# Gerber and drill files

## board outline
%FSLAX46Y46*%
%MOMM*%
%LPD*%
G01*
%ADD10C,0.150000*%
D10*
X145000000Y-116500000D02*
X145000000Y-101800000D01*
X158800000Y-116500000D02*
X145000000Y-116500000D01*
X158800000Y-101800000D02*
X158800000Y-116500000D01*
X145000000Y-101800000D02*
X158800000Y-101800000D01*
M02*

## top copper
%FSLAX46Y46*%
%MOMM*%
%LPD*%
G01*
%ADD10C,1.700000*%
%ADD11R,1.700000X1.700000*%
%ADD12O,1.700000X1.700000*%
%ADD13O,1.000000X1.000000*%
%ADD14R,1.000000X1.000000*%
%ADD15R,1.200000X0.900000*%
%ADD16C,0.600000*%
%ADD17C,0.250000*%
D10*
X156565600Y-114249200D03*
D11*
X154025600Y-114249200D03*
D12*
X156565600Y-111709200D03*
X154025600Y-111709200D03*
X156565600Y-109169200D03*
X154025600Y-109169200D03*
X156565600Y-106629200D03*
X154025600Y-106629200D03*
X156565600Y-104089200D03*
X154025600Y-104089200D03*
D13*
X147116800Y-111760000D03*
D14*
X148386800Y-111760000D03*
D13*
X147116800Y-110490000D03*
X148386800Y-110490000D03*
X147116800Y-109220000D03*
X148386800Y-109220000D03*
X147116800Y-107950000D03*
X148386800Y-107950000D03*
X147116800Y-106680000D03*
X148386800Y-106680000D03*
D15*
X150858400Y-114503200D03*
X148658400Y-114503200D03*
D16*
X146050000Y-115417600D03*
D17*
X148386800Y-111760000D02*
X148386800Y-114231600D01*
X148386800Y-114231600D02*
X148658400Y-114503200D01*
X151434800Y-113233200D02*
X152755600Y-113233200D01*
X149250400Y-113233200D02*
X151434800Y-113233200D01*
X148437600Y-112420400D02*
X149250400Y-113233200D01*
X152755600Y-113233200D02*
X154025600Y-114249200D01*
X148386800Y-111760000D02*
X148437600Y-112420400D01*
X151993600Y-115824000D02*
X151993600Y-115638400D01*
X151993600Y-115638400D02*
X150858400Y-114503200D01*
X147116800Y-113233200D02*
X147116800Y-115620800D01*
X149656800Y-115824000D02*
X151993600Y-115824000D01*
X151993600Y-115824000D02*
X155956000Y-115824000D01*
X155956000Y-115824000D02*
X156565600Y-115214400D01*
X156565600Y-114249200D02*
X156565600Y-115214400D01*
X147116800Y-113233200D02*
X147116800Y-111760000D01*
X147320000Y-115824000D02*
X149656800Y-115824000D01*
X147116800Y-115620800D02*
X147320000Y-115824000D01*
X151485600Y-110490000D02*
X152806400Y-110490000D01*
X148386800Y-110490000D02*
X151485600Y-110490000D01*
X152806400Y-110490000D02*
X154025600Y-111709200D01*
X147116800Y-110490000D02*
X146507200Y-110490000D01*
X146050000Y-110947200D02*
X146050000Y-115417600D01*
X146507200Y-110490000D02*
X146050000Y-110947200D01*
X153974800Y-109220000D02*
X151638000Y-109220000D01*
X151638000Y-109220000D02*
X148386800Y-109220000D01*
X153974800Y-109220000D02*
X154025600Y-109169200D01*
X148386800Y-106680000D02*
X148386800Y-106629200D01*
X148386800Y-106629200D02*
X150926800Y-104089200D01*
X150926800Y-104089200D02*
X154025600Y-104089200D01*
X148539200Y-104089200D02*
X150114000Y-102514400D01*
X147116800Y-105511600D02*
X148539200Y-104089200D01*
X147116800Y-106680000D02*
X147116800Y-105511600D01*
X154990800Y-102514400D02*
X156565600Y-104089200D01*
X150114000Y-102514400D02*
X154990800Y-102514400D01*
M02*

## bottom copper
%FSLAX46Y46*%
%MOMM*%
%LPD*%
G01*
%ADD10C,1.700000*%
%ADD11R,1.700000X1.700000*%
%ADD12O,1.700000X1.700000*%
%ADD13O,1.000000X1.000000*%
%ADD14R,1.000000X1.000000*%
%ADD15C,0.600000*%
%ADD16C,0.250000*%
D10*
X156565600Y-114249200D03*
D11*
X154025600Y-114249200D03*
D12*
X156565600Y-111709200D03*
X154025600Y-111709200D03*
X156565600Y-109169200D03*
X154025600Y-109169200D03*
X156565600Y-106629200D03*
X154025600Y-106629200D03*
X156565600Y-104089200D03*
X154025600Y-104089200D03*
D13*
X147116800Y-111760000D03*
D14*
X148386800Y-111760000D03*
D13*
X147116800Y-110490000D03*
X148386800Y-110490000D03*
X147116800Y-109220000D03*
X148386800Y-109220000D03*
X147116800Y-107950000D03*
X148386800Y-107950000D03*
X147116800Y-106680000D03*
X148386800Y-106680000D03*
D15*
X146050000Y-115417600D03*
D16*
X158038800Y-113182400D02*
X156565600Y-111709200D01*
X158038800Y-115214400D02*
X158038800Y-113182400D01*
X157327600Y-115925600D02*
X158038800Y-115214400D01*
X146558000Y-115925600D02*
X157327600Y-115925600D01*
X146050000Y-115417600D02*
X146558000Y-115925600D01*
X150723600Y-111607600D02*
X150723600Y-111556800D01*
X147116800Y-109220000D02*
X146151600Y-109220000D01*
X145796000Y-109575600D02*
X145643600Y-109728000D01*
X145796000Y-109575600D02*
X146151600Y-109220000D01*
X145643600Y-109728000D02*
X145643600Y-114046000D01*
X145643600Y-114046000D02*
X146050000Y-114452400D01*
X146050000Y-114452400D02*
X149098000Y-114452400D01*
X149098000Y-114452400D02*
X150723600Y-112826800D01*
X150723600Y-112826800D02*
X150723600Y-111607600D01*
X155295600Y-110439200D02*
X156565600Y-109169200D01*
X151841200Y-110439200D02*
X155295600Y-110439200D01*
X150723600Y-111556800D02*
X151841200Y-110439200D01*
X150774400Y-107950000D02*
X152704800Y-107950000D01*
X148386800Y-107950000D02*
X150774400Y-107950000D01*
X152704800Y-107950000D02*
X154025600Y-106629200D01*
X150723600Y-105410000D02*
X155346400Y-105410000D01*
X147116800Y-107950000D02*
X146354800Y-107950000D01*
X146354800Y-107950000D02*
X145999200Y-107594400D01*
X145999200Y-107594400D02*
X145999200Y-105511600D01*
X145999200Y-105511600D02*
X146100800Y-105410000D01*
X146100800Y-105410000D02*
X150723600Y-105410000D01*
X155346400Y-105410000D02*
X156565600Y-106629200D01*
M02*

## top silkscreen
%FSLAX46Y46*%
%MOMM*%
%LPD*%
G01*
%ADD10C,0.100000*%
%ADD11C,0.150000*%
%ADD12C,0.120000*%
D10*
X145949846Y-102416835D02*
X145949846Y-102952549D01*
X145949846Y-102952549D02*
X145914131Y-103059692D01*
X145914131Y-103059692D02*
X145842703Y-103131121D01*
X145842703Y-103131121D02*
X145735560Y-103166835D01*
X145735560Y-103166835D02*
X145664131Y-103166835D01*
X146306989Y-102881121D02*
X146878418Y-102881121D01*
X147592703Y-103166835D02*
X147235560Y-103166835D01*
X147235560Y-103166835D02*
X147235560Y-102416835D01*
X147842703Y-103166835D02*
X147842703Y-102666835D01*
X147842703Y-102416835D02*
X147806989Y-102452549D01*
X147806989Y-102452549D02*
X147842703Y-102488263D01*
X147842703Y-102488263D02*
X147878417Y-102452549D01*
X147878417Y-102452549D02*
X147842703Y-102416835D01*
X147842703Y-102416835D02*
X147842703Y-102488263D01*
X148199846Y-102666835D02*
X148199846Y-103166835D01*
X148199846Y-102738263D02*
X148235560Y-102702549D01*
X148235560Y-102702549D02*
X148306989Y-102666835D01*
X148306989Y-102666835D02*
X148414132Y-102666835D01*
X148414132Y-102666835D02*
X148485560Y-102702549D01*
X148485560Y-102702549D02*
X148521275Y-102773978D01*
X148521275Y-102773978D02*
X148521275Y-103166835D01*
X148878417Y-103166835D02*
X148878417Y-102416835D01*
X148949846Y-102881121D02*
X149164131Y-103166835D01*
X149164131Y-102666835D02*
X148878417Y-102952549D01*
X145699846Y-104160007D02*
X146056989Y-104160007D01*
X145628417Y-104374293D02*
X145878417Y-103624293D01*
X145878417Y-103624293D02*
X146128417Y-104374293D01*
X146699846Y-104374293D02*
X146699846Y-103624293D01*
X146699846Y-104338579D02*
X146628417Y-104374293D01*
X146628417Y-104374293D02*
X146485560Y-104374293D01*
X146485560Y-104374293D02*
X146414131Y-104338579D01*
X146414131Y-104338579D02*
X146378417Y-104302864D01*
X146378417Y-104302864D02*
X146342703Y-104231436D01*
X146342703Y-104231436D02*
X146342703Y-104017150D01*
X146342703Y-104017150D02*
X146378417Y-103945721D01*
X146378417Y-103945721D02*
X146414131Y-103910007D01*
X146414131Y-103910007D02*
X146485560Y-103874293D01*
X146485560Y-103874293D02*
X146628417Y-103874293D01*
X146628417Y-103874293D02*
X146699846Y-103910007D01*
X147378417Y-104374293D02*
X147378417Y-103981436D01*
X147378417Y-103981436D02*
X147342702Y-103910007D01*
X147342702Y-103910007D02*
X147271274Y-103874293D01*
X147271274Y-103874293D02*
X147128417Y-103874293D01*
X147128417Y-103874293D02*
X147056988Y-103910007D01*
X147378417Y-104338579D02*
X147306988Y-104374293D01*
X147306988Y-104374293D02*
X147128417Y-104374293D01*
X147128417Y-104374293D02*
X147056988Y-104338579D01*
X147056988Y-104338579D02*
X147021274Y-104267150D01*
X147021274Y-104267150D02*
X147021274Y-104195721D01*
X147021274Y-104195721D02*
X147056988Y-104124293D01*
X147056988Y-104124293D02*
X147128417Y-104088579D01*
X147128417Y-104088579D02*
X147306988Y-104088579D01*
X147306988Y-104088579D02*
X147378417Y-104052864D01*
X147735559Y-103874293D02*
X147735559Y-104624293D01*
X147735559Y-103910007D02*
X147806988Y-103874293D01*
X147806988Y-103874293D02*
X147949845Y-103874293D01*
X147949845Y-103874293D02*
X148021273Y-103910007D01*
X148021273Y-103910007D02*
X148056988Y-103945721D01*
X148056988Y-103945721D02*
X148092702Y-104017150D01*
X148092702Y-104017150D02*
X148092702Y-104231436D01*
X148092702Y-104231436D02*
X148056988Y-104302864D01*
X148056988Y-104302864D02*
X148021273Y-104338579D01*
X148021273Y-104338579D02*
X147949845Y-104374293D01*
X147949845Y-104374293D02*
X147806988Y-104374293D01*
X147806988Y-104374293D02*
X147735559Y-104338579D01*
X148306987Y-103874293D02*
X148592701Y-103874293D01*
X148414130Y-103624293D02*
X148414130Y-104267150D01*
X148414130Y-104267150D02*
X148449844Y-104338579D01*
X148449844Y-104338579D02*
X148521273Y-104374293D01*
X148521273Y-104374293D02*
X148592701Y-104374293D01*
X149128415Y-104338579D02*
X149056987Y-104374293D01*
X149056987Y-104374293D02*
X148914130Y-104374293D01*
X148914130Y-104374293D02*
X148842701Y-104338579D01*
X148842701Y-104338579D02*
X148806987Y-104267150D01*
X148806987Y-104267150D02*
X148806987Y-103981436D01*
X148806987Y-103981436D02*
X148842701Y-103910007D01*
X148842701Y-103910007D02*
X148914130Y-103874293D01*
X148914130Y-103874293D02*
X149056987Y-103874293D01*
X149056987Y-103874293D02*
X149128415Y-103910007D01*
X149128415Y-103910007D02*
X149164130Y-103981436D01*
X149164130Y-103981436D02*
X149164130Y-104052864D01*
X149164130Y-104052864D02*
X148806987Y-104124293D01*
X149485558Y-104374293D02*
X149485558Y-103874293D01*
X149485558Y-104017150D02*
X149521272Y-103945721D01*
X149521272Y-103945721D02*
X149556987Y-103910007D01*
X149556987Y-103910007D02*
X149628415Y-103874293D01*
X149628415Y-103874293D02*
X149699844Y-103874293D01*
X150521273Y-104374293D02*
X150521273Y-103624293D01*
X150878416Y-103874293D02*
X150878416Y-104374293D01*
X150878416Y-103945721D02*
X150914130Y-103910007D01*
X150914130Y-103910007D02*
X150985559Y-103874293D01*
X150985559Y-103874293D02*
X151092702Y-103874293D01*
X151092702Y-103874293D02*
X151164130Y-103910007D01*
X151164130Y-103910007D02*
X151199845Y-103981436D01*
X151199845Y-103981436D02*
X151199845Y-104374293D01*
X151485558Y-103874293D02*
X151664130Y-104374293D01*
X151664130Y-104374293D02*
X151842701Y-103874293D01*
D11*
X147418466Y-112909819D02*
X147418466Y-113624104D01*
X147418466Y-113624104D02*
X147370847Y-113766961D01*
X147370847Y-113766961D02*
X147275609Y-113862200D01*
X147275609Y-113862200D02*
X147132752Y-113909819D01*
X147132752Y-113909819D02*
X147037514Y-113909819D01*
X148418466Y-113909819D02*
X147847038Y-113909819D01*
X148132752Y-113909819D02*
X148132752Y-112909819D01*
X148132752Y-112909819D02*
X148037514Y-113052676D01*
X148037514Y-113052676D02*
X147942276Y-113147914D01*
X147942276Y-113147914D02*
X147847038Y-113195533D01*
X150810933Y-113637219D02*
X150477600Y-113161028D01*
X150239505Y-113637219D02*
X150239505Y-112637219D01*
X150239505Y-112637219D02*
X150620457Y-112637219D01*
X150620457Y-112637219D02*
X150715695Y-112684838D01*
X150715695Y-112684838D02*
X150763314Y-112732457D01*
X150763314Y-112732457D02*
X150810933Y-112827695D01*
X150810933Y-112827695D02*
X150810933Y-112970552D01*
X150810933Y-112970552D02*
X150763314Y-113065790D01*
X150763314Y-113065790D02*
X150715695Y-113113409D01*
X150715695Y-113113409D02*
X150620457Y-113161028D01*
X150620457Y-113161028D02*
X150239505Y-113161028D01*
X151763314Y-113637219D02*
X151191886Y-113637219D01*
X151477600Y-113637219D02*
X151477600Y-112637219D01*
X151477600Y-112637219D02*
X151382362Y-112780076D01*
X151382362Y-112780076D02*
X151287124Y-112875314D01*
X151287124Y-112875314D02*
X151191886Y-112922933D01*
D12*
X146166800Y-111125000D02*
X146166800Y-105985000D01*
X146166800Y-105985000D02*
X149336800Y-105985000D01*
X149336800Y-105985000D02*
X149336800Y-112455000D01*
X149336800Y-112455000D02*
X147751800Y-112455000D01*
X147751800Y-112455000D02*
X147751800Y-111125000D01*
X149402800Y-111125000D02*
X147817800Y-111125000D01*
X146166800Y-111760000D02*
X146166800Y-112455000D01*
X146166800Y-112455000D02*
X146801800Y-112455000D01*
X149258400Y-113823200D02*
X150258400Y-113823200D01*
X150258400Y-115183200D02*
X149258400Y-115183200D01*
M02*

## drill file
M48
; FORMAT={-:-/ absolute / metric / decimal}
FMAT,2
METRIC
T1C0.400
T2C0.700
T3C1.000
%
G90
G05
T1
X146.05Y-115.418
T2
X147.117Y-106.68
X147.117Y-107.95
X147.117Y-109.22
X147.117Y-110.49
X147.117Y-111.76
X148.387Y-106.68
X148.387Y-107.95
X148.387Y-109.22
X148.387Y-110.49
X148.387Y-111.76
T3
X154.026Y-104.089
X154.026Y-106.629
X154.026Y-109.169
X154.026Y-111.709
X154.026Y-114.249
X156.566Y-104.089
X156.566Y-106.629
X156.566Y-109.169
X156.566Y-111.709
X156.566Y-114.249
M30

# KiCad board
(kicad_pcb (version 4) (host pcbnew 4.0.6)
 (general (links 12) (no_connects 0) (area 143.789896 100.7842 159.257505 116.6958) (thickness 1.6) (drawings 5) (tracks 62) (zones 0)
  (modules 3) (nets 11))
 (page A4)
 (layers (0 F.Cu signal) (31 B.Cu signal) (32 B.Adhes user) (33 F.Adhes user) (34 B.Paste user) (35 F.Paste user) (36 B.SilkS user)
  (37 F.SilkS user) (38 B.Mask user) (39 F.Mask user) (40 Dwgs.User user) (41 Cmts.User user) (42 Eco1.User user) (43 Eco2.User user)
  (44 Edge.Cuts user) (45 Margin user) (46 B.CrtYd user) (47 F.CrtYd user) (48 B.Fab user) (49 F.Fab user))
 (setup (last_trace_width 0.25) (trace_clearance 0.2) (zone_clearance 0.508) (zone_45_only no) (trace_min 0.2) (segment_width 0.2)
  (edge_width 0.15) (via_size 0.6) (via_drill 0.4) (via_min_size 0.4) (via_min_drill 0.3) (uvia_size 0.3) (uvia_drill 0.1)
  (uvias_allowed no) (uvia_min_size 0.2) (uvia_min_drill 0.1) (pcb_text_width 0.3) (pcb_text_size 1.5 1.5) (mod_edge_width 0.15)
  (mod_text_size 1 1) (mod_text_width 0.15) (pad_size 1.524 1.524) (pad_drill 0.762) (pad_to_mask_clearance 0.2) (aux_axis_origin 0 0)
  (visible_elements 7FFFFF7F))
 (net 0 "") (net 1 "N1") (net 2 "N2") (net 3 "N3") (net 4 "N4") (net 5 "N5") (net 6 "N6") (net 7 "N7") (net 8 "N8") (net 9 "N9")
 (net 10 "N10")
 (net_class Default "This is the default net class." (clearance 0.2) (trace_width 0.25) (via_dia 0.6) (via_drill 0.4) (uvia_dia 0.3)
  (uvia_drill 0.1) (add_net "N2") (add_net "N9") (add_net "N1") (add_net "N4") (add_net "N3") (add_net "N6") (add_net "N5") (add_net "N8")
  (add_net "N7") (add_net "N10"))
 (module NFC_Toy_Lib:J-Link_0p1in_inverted (layer B.Cu) (at 156.5656 114.2492)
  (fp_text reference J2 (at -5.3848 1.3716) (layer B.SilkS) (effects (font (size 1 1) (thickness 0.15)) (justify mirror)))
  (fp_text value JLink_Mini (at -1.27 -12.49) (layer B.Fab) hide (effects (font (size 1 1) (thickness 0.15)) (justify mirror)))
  (pad 2 thru_hole circle (at 0 0) (size 1.7 1.7) (drill 1) (layers *.Cu *.Mask) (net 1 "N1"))
  (pad 1 thru_hole rect (at -2.54 0) (size 1.7 1.7) (drill 1) (layers *.Cu *.Mask) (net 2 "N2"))
  (pad 4 thru_hole oval (at 0 -2.54) (size 1.7 1.7) (drill 1) (layers *.Cu *.Mask) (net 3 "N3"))
  (pad 3 thru_hole oval (at -2.54 -2.54) (size 1.7 1.7) (drill 1) (layers *.Cu *.Mask) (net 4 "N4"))
  (pad 6 thru_hole oval (at 0 -5.08) (size 1.7 1.7) (drill 1) (layers *.Cu *.Mask) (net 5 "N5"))
  (pad 5 thru_hole oval (at -2.54 -5.08) (size 1.7 1.7) (drill 1) (layers *.Cu *.Mask) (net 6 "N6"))
  (pad 8 thru_hole oval (at 0 -7.62) (size 1.7 1.7) (drill 1) (layers *.Cu *.Mask) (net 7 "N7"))
  (pad 7 thru_hole oval (at -2.54 -7.62) (size 1.7 1.7) (drill 1) (layers *.Cu *.Mask) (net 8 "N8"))
  (pad 10 thru_hole oval (at 0 -10.16) (size 1.7 1.7) (drill 1) (layers *.Cu *.Mask) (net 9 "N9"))
  (pad 9 thru_hole oval (at -2.54 -10.16) (size 1.7 1.7) (drill 1) (layers *.Cu *.Mask) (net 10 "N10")))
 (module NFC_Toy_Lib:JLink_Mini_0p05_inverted (layer F.Cu) (at 147.1168 111.76 180)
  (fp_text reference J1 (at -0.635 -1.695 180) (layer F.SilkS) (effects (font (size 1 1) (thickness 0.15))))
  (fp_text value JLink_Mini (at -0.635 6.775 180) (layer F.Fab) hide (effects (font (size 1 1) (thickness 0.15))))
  (fp_line (start 0.95 0.635) (end 0.95 5.775) (layer F.SilkS) (width 0.12))
  (fp_line (start 0.95 5.775) (end -2.22 5.775) (layer F.SilkS) (width 0.12))
  (fp_line (start -2.22 5.775) (end -2.22 -0.695) (layer F.SilkS) (width 0.12))
  (fp_line (start -2.22 -0.695) (end -0.635 -0.695) (layer F.SilkS) (width 0.12))
  (fp_line (start -0.635 -0.695) (end -0.635 0.635) (layer F.SilkS) (width 0.12))
  (fp_line (start -2.286 0.635) (end -0.701 0.635) (layer F.SilkS) (width 0.12))
  (fp_line (start 0.95 0) (end 0.95 -0.695) (layer F.SilkS) (width 0.12))
  (fp_line (start 0.95 -0.695) (end 0.315 -0.695) (layer F.SilkS) (width 0.12))
  (pad 2 thru_hole oval (at 0 0 180) (size 1 1) (drill 0.7) (layers *.Cu *.Mask) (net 1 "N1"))
  (pad 1 thru_hole rect (at -1.27 0 180) (size 1 1) (drill 0.7) (layers *.Cu *.Mask) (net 2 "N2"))
  (pad 4 thru_hole oval (at 0 1.27 180) (size 1 1) (drill 0.7) (layers *.Cu *.Mask) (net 3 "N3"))
  (pad 3 thru_hole oval (at -1.27 1.27 180) (size 1 1) (drill 0.7) (layers *.Cu *.Mask) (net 4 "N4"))
  (pad 6 thru_hole oval (at 0 2.54 180) (size 1 1) (drill 0.7) (layers *.Cu *.Mask) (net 5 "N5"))
  (pad 5 thru_hole oval (at -1.27 2.54 180) (size 1 1) (drill 0.7) (layers *.Cu *.Mask) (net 6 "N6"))
  (pad 8 thru_hole oval (at 0 3.81 180) (size 1 1) (drill 0.7) (layers *.Cu *.Mask) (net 7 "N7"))
  (pad 7 thru_hole oval (at -1.27 3.81 180) (size 1 1) (drill 0.7) (layers *.Cu *.Mask) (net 8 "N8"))
  (pad 10 thru_hole oval (at 0 5.08 180) (size 1 1) (drill 0.7) (layers *.Cu *.Mask) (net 9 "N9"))
  (pad 9 thru_hole oval (at -1.27 5.08 180) (size 1 1) (drill 0.7) (layers *.Cu *.Mask) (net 10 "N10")))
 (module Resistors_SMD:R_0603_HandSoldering (layer F.Cu) (at 149.7584 114.5032 180)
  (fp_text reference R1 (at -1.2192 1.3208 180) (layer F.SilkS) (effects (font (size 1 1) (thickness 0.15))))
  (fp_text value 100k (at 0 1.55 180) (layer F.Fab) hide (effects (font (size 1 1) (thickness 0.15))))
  (fp_line (start 0.5 0.68) (end -0.5 0.68) (layer F.SilkS) (width 0.12))
  (fp_line (start -0.5 -0.68) (end 0.5 -0.68) (layer F.SilkS) (width 0.12))
  (pad 1 smd rect (at -1.1 0 180) (size 1.2 0.9) (layers F.Cu F.Paste F.Mask) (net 1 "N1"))
  (pad 2 smd rect (at 1.1 0 180) (size 1.2 0.9) (layers F.Cu F.Paste F.Mask) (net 2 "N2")))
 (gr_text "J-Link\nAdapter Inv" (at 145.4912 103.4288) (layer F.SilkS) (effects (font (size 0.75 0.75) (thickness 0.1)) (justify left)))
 (gr_line (start 145 116.5) (end 145 101.8) (angle 90) (layer Edge.Cuts) (width 0.15))
 (gr_line (start 158.8 116.5) (end 145 116.5) (angle 90) (layer Edge.Cuts) (width 0.15))
 (gr_line (start 158.8 101.8) (end 158.8 116.5) (angle 90) (layer Edge.Cuts) (width 0.15))
 (gr_line (start 145 101.8) (end 158.8 101.8) (angle 90) (layer Edge.Cuts) (width 0.15))
 (segment (start 148.3868 111.76) (end 148.3868 114.2316) (width 0.25) (layer F.Cu) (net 2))
 (segment (start 148.3868 114.2316) (end 148.6584 114.5032) (width 0.25) (layer F.Cu) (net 2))
 (segment (start 151.4348 113.2332) (end 152.7556 113.2332) (width 0.25) (layer F.Cu) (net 2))
 (segment (start 149.2504 113.2332) (end 151.4348 113.2332) (width 0.25) (layer F.Cu) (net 2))
 (segment (start 148.4376 112.4204) (end 149.2504 113.2332) (width 0.25) (layer F.Cu) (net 2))
 (segment (start 152.7556 113.2332) (end 154.0256 114.2492) (width 0.25) (layer F.Cu) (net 2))
 (segment (start 148.3868 111.76) (end 148.4376 112.4204) (width 0.25) (layer F.Cu) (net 2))
 (segment (start 151.9936 115.824) (end 151.9936 115.6384) (width 0.25) (layer F.Cu) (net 1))
 (segment (start 151.9936 115.6384) (end 150.8584 114.5032) (width 0.25) (layer F.Cu) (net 1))
 (segment (start 147.1168 113.2332) (end 147.1168 115.6208) (width 0.25) (layer F.Cu) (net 1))
 (segment (start 149.6568 115.824) (end 151.9936 115.824) (width 0.25) (layer F.Cu) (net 1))
 (segment (start 151.9936 115.824) (end 155.956 115.824) (width 0.25) (layer F.Cu) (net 1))
 (segment (start 155.956 115.824) (end 156.5656 115.2144) (width 0.25) (layer F.Cu) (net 1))
 (segment (start 156.5656 114.2492) (end 156.5656 115.2144) (width 0.25) (layer F.Cu) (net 1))
 (segment (start 147.1168 113.2332) (end 147.1168 111.76) (width 0.25) (layer F.Cu) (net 1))
 (segment (start 147.32 115.824) (end 149.6568 115.824) (width 0.25) (layer F.Cu) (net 1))
 (segment (start 147.1168 115.6208) (end 147.32 115.824) (width 0.25) (layer F.Cu) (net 1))
 (segment (start 151.4856 110.49) (end 152.8064 110.49) (width 0.25) (layer F.Cu) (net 4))
 (segment (start 148.3868 110.49) (end 151.4856 110.49) (width 0.25) (layer F.Cu) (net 4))
 (segment (start 152.8064 110.49) (end 154.0256 111.7092) (width 0.25) (layer F.Cu) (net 4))
 (segment (start 147.1168 110.49) (end 146.5072 110.49) (width 0.25) (layer F.Cu) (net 3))
 (segment (start 158.0388 113.1824) (end 156.5656 111.7092) (width 0.25) (layer B.Cu) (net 3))
 (segment (start 158.0388 115.2144) (end 158.0388 113.1824) (width 0.25) (layer B.Cu) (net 3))
 (segment (start 157.3276 115.9256) (end 158.0388 115.2144) (width 0.25) (layer B.Cu) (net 3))
 (segment (start 146.558 115.9256) (end 157.3276 115.9256) (width 0.25) (layer B.Cu) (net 3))
 (segment (start 146.05 115.4176) (end 146.558 115.9256) (width 0.25) (layer B.Cu) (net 3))
 (via (at 146.05 115.4176) (size 0.6) (drill 0.4) (layers F.Cu B.Cu) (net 3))
 (segment (start 146.05 110.9472) (end 146.05 115.4176) (width 0.25) (layer F.Cu) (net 3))
 (segment (start 146.5072 110.49) (end 146.05 110.9472) (width 0.25) (layer F.Cu) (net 3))
 (segment (start 153.9748 109.22) (end 151.638 109.22) (width 0.25) (layer F.Cu) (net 6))
 (segment (start 151.638 109.22) (end 148.3868 109.22) (width 0.25) (layer F.Cu) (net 6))
 (segment (start 153.9748 109.22) (end 154.0256 109.1692) (width 0.25) (layer F.Cu) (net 6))
 (segment (start 150.7236 111.6076) (end 150.7236 111.5568) (width 0.25) (layer B.Cu) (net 5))
 (segment (start 147.1168 109.22) (end 146.1516 109.22) (width 0.25) (layer B.Cu) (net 5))
 (segment (start 145.796 109.5756) (end 145.6436 109.728) (width 0.25) (layer B.Cu) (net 5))
 (segment (start 145.796 109.5756) (end 146.1516 109.22) (width 0.25) (layer B.Cu) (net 5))
 (segment (start 145.6436 109.728) (end 145.6436 114.046) (width 0.25) (layer B.Cu) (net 5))
 (segment (start 145.6436 114.046) (end 146.05 114.4524) (width 0.25) (layer B.Cu) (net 5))
 (segment (start 146.05 114.4524) (end 149.098 114.4524) (width 0.25) (layer B.Cu) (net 5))
 (segment (start 149.098 114.4524) (end 150.7236 112.8268) (width 0.25) (layer B.Cu) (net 5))
 (segment (start 150.7236 112.8268) (end 150.7236 111.6076) (width 0.25) (layer B.Cu) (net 5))
 (segment (start 155.2956 110.4392) (end 156.5656 109.1692) (width 0.25) (layer B.Cu) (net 5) (status 800000))
 (segment (start 151.8412 110.4392) (end 155.2956 110.4392) (width 0.25) (layer B.Cu) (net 5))
 (segment (start 150.7236 111.5568) (end 151.8412 110.4392) (width 0.25) (layer B.Cu) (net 5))
 (segment (start 150.7744 107.95) (end 152.7048 107.95) (width 0.25) (layer B.Cu) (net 8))
 (segment (start 148.3868 107.95) (end 150.7744 107.95) (width 0.25) (layer B.Cu) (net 8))
 (segment (start 152.7048 107.95) (end 154.0256 106.6292) (width 0.25) (layer B.Cu) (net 8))
 (segment (start 150.7236 105.41) (end 155.3464 105.41) (width 0.25) (layer B.Cu) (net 7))
 (segment (start 147.1168 107.95) (end 146.3548 107.95) (width 0.25) (layer B.Cu) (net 7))
 (segment (start 146.3548 107.95) (end 145.9992 107.5944) (width 0.25) (layer B.Cu) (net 7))
 (segment (start 145.9992 107.5944) (end 145.9992 105.5116) (width 0.25) (layer B.Cu) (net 7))
 (segment (start 145.9992 105.5116) (end 146.1008 105.41) (width 0.25) (layer B.Cu) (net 7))
 (segment (start 146.1008 105.41) (end 150.7236 105.41) (width 0.25) (layer B.Cu) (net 7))
 (segment (start 155.3464 105.41) (end 156.5656 106.6292) (width 0.25) (layer B.Cu) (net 7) (status 800000))
 (segment (start 148.3868 106.68) (end 148.3868 106.6292) (width 0.25) (layer F.Cu) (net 10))
 (segment (start 148.3868 106.6292) (end 150.9268 104.0892) (width 0.25) (layer F.Cu) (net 10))
 (segment (start 150.9268 104.0892) (end 154.0256 104.0892) (width 0.25) (layer F.Cu) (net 10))
 (segment (start 148.5392 104.0892) (end 150.114 102.5144) (width 0.25) (layer F.Cu) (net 9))
 (segment (start 147.1168 105.5116) (end 148.5392 104.0892) (width 0.25) (layer F.Cu) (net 9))
 (segment (start 147.1168 106.68) (end 147.1168 105.5116) (width 0.25) (layer F.Cu) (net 9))
 (segment (start 154.9908 102.5144) (end 156.5656 104.0892) (width 0.25) (layer F.Cu) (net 9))
 (segment (start 150.114 102.5144) (end 154.9908 102.5144) (width 0.25) (layer F.Cu) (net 9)))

